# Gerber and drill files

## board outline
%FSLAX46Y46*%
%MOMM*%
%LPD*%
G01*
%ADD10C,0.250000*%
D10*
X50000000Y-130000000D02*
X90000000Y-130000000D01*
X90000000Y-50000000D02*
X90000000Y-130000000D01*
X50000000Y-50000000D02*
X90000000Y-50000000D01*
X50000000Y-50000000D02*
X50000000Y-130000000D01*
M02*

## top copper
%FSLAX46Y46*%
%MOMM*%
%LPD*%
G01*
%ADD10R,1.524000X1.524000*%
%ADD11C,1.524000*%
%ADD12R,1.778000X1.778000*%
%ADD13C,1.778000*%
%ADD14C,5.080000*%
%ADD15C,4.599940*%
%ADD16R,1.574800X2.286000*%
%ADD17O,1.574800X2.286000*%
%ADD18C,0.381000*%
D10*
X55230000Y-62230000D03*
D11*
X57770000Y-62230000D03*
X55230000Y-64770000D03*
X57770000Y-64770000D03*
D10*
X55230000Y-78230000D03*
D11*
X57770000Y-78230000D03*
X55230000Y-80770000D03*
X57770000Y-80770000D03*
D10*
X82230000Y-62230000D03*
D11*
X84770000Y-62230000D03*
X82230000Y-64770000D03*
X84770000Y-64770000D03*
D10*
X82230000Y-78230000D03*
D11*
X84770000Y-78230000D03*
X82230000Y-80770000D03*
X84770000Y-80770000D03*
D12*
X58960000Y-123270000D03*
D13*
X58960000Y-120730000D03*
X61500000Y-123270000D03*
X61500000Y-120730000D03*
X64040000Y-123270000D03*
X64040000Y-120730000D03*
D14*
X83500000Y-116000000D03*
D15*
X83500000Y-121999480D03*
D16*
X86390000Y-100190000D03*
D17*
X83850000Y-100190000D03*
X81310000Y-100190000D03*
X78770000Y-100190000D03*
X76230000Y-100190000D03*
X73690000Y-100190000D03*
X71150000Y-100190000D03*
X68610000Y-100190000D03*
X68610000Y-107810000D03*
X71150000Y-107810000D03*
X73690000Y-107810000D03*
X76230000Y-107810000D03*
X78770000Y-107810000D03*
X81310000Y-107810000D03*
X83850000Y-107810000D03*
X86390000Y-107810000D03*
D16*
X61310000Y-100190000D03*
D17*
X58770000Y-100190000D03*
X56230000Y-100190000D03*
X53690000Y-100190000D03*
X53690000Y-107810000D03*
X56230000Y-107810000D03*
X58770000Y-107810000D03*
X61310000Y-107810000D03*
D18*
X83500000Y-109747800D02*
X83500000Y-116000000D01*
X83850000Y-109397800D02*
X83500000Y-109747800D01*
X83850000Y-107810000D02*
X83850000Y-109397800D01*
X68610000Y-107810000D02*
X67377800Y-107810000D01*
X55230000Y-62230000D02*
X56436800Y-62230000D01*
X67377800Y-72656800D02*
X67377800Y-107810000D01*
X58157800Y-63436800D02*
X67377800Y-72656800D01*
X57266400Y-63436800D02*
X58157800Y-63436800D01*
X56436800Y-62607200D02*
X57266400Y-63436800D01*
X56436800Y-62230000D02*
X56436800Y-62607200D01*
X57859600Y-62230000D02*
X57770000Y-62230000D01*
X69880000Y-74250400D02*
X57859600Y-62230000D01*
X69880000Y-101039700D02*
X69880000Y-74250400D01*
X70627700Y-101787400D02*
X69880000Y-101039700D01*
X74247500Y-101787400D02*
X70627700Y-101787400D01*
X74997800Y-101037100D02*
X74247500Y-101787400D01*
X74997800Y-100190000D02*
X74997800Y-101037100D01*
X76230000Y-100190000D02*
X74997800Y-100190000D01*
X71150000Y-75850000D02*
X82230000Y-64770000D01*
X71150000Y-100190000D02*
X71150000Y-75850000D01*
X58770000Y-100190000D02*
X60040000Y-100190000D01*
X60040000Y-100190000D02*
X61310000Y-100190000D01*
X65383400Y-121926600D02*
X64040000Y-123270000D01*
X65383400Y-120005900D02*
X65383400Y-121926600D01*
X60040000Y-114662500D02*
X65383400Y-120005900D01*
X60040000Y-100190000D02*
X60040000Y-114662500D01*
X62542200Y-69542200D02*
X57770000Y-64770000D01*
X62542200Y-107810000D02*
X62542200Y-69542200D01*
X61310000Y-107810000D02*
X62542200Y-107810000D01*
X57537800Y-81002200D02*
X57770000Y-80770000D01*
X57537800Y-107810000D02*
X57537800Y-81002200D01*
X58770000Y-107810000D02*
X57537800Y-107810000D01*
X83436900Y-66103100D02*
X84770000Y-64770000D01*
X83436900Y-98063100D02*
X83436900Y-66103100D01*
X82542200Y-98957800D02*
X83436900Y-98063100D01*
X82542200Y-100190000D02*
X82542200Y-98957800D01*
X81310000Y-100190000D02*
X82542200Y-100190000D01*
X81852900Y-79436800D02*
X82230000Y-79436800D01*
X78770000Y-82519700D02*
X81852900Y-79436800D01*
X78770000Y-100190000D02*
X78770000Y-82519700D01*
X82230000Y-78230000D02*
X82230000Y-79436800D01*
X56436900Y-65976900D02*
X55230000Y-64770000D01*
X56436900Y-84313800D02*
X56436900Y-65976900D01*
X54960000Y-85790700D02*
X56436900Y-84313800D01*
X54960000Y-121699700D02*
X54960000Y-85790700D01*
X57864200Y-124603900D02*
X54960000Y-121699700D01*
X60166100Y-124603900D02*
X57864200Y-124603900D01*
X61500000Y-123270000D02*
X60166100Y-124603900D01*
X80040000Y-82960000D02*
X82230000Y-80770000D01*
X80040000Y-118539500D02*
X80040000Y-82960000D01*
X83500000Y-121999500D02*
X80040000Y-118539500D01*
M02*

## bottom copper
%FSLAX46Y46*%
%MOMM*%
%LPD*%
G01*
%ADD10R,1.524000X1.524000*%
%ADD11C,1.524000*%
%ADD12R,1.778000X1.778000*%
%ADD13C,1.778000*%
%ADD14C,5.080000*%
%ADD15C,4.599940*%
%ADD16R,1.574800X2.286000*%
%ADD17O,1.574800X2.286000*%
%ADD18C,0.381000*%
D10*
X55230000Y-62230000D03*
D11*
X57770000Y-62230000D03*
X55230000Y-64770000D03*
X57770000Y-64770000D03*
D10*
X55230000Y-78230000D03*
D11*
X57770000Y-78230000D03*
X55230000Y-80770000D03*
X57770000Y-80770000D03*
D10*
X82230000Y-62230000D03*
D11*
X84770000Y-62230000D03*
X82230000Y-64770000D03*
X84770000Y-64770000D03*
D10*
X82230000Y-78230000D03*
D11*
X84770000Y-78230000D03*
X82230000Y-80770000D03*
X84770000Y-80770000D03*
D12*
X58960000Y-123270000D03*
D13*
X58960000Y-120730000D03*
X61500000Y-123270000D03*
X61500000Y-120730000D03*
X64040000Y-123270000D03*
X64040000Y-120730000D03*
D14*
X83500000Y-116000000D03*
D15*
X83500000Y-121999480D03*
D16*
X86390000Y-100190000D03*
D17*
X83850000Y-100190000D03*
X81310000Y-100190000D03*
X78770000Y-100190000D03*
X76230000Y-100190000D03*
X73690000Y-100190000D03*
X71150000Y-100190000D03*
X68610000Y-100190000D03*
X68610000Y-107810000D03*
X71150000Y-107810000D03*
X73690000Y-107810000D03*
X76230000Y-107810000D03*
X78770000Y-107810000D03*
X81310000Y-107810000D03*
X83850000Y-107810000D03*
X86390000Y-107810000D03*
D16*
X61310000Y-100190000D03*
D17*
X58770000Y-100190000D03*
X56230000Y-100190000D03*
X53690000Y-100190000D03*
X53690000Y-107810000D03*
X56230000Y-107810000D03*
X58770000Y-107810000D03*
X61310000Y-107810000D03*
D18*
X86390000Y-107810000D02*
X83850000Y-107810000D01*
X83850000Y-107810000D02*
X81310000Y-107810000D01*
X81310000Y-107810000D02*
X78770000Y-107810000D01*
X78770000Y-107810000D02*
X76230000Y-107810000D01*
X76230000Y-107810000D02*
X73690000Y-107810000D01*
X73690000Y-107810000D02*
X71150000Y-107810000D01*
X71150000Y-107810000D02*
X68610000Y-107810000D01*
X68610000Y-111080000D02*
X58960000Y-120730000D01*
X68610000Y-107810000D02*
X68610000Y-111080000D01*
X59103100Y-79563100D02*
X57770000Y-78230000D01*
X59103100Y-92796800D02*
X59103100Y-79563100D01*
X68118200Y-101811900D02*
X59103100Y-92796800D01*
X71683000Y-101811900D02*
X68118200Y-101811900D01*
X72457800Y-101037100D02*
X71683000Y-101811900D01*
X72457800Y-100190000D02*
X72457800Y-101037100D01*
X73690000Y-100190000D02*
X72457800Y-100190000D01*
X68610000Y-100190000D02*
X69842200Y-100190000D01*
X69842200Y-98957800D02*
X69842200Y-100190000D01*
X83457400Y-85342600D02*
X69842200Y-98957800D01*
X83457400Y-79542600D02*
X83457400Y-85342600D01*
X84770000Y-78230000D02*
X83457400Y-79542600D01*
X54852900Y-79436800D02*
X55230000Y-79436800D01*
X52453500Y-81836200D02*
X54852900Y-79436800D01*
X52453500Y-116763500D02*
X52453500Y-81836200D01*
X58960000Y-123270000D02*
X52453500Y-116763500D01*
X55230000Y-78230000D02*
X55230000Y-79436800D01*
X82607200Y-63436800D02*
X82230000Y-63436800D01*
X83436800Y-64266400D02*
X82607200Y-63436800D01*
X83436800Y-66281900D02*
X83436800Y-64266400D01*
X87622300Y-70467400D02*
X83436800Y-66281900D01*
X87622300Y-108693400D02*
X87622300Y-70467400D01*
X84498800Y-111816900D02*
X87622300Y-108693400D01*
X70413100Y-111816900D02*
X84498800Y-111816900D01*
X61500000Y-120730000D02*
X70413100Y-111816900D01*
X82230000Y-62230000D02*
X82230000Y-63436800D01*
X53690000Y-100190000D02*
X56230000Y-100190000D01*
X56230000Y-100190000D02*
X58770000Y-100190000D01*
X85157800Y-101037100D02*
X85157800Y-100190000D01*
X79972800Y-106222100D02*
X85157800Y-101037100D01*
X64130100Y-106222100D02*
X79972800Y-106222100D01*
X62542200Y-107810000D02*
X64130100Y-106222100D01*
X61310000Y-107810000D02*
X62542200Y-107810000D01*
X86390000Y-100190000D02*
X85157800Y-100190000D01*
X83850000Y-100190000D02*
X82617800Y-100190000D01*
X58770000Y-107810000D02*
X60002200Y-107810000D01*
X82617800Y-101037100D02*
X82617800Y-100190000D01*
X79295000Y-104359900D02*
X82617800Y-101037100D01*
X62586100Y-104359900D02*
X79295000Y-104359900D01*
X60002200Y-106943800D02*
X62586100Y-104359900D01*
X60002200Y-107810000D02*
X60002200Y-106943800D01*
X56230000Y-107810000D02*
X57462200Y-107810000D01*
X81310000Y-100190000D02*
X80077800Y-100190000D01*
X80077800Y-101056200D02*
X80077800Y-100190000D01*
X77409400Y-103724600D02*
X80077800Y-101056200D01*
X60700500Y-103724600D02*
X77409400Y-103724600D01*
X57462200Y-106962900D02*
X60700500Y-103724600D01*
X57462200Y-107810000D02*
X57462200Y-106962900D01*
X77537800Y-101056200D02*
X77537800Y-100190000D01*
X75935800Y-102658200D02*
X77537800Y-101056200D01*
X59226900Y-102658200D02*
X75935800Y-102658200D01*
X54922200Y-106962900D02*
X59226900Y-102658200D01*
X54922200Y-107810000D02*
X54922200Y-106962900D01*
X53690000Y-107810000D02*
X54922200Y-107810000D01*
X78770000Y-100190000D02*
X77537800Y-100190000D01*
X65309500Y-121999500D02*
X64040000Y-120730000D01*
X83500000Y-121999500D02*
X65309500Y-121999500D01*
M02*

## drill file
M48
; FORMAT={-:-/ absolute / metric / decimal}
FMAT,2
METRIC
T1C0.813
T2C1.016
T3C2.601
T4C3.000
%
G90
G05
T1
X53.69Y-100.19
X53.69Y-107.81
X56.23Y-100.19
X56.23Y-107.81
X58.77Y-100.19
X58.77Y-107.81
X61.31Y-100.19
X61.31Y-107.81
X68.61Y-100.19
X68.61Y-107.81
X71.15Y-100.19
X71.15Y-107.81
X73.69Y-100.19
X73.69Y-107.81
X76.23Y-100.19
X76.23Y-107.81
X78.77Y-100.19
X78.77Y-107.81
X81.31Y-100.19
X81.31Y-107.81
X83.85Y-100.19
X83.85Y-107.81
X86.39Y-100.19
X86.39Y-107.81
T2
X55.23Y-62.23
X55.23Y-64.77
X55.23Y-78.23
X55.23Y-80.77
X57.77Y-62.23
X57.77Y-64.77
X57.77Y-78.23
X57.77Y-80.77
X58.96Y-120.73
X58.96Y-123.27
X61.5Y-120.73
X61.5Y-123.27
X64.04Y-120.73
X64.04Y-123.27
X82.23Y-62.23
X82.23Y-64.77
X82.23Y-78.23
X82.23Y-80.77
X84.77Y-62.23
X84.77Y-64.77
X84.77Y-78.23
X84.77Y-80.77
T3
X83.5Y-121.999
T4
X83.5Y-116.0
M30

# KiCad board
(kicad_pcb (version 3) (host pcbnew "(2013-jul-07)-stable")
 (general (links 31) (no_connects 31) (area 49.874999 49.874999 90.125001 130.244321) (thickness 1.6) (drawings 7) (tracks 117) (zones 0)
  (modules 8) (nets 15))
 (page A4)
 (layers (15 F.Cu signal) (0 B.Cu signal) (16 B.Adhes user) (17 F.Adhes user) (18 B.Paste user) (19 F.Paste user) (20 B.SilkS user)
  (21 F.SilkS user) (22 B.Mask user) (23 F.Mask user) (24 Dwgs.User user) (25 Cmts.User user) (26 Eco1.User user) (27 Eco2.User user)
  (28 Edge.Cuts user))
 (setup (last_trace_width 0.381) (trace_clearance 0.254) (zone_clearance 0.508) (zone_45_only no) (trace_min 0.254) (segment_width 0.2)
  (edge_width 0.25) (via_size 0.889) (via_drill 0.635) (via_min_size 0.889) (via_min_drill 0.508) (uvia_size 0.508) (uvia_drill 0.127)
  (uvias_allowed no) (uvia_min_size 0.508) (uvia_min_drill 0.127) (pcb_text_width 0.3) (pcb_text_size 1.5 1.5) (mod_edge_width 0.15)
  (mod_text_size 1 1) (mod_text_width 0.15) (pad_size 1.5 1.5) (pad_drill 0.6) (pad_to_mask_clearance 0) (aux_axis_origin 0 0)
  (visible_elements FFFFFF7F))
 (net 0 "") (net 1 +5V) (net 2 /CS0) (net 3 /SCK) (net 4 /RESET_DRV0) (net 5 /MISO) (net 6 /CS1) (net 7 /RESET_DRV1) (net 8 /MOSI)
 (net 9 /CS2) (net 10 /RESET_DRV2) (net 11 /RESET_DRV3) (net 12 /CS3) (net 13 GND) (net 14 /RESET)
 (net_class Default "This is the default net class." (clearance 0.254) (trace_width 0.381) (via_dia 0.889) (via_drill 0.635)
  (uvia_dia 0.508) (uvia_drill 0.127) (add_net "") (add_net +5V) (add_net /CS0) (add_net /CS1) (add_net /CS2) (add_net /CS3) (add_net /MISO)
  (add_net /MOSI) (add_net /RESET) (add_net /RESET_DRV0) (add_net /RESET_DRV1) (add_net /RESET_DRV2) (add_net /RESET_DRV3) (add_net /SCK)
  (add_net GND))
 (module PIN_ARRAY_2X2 (layer F.Cu) (at 56.5 63.5 270)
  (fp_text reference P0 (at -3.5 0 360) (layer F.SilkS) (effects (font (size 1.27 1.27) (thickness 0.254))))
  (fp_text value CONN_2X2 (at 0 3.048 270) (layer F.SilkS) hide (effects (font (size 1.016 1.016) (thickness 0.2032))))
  (pad 1 thru_hole rect (at -1.27 1.27 270) (size 1.524 1.524) (drill 1.016) (layers *.Cu *.Mask F.SilkS) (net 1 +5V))
  (pad 2 thru_hole circle (at -1.27 -1.27 270) (size 1.524 1.524) (drill 1.016) (layers *.Cu *.Mask F.SilkS) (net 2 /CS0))
  (pad 3 thru_hole circle (at 1.27 1.27 270) (size 1.524 1.524) (drill 1.016) (layers *.Cu *.Mask F.SilkS) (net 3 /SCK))
  (pad 4 thru_hole circle (at 1.27 -1.27 270) (size 1.524 1.524) (drill 1.016) (layers *.Cu *.Mask F.SilkS) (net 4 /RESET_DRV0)))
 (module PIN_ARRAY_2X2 (layer F.Cu) (at 56.5 79.5 270)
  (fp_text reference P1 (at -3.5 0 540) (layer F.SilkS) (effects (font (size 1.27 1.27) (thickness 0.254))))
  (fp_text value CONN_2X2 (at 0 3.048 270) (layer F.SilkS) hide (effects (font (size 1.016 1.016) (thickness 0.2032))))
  (pad 1 thru_hole rect (at -1.27 1.27 270) (size 1.524 1.524) (drill 1.016) (layers *.Cu *.Mask F.SilkS) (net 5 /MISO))
  (pad 2 thru_hole circle (at -1.27 -1.27 270) (size 1.524 1.524) (drill 1.016) (layers *.Cu *.Mask F.SilkS) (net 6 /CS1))
  (pad 3 thru_hole circle (at 1.27 1.27 270) (size 1.524 1.524) (drill 1.016) (layers *.Cu *.Mask F.SilkS))
  (pad 4 thru_hole circle (at 1.27 -1.27 270) (size 1.524 1.524) (drill 1.016) (layers *.Cu *.Mask F.SilkS) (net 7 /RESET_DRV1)))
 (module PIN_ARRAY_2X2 (layer F.Cu) (at 83.5 63.5 270)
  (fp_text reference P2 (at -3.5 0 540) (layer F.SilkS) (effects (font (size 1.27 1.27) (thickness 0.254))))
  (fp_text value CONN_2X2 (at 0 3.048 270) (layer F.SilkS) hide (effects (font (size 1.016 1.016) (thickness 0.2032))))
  (pad 1 thru_hole rect (at -1.27 1.27 270) (size 1.524 1.524) (drill 1.016) (layers *.Cu *.Mask F.SilkS) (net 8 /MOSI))
  (pad 2 thru_hole circle (at -1.27 -1.27 270) (size 1.524 1.524) (drill 1.016) (layers *.Cu *.Mask F.SilkS))
  (pad 3 thru_hole circle (at 1.27 1.27 270) (size 1.524 1.524) (drill 1.016) (layers *.Cu *.Mask F.SilkS) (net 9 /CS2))
  (pad 4 thru_hole circle (at 1.27 -1.27 270) (size 1.524 1.524) (drill 1.016) (layers *.Cu *.Mask F.SilkS) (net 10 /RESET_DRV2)))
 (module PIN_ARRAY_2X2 (layer F.Cu) (at 83.5 79.5 270)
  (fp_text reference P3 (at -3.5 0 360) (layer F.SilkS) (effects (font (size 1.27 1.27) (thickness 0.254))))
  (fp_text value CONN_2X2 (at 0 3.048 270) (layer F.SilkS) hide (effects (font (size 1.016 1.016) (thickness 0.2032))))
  (pad 1 thru_hole rect (at -1.27 1.27 270) (size 1.524 1.524) (drill 1.016) (layers *.Cu *.Mask F.SilkS) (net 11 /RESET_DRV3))
  (pad 2 thru_hole circle (at -1.27 -1.27 270) (size 1.524 1.524) (drill 1.016) (layers *.Cu *.Mask F.SilkS) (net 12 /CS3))
  (pad 3 thru_hole circle (at 1.27 1.27 270) (size 1.524 1.524) (drill 1.016) (layers *.Cu *.Mask F.SilkS) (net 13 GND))
  (pad 4 thru_hole circle (at 1.27 -1.27 270) (size 1.524 1.524) (drill 1.016) (layers *.Cu *.Mask F.SilkS)))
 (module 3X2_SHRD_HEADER (layer F.Cu) (at 61.5 122)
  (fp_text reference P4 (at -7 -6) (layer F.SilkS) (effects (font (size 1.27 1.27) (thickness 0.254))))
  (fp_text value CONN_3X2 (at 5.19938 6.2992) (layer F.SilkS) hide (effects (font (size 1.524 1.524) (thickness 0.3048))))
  (pad 1 thru_hole rect (at -2.54 1.27) (size 1.778 1.778) (drill 1.016) (layers *.Cu *.Mask F.SilkS) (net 5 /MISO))
  (pad 2 thru_hole circle (at -2.54 -1.27) (size 1.778 1.778) (drill 1.016) (layers *.Cu *.Mask F.SilkS) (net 1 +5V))
  (pad 3 thru_hole circle (at 0 1.27) (size 1.778 1.778) (drill 1.016) (layers *.Cu *.Mask F.SilkS) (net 3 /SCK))
  (pad 4 thru_hole circle (at 0 -1.27) (size 1.778 1.778) (drill 1.016) (layers *.Cu *.Mask F.SilkS) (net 8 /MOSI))
  (pad 5 thru_hole circle (at 2.54 1.27) (size 1.778 1.778) (drill 1.016) (layers *.Cu *.Mask F.SilkS) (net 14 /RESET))
  (pad 6 thru_hole circle (at 2.54 -1.27) (size 1.778 1.778) (drill 1.016) (layers *.Cu *.Mask F.SilkS) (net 13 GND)))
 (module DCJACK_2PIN (layer F.Cu) (at 83.5 116 270)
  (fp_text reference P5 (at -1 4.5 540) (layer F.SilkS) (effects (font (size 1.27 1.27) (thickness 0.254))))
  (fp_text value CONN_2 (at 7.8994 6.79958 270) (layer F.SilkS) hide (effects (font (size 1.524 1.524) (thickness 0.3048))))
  (pad 1 thru_hole circle (at 0 0 270) (size 5.08 5.08) (drill 2.99974) (layers *.Cu *.Mask F.SilkS) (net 1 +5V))
  (pad 2 thru_hole circle (at 5.99948 0 270) (size 4.59994 4.59994) (drill 2.60096) (layers *.Cu *.Mask F.SilkS) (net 13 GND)))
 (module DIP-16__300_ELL (layer F.Cu) (at 77.5 104 180)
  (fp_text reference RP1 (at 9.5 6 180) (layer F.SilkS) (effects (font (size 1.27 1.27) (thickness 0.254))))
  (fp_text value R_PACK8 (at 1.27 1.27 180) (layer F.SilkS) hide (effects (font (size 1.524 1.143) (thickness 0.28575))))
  (pad 1 thru_hole rect (at -8.89 3.81 180) (size 1.5748 2.286) (drill 0.8128) (layers *.Cu *.Mask F.SilkS) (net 4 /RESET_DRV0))
  (pad 2 thru_hole oval (at -6.35 3.81 180) (size 1.5748 2.286) (drill 0.8128) (layers *.Cu *.Mask F.SilkS) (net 7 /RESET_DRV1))
  (pad 3 thru_hole oval (at -3.81 3.81 180) (size 1.5748 2.286) (drill 0.8128) (layers *.Cu *.Mask F.SilkS) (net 10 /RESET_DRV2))
  (pad 4 thru_hole oval (at -1.27 3.81 180) (size 1.5748 2.286) (drill 0.8128) (layers *.Cu *.Mask F.SilkS) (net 11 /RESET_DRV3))
  (pad 5 thru_hole oval (at 1.27 3.81 180) (size 1.5748 2.286) (drill 0.8128) (layers *.Cu *.Mask F.SilkS) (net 2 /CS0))
  (pad 6 thru_hole oval (at 3.81 3.81 180) (size 1.5748 2.286) (drill 0.8128) (layers *.Cu *.Mask F.SilkS) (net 6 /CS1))
  (pad 7 thru_hole oval (at 6.35 3.81 180) (size 1.5748 2.286) (drill 0.8128) (layers *.Cu *.Mask F.SilkS) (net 9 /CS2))
  (pad 8 thru_hole oval (at 8.89 3.81 180) (size 1.5748 2.286) (drill 0.8128) (layers *.Cu *.Mask F.SilkS) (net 12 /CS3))
  (pad 9 thru_hole oval (at 8.89 -3.81 180) (size 1.5748 2.286) (drill 0.8128) (layers *.Cu *.Mask F.SilkS) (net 1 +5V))
  (pad 10 thru_hole oval (at 6.35 -3.81 180) (size 1.5748 2.286) (drill 0.8128) (layers *.Cu *.Mask F.SilkS) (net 1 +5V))
  (pad 11 thru_hole oval (at 3.81 -3.81 180) (size 1.5748 2.286) (drill 0.8128) (layers *.Cu *.Mask F.SilkS) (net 1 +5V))
  (pad 12 thru_hole oval (at 1.27 -3.81 180) (size 1.5748 2.286) (drill 0.8128) (layers *.Cu *.Mask F.SilkS) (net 1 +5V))
  (pad 13 thru_hole oval (at -1.27 -3.81 180) (size 1.5748 2.286) (drill 0.8128) (layers *.Cu *.Mask F.SilkS) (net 1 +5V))
  (pad 14 thru_hole oval (at -3.81 -3.81 180) (size 1.5748 2.286) (drill 0.8128) (layers *.Cu *.Mask F.SilkS) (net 1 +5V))
  (pad 15 thru_hole oval (at -6.35 -3.81 180) (size 1.5748 2.286) (drill 0.8128) (layers *.Cu *.Mask F.SilkS) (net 1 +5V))
  (pad 16 thru_hole oval (at -8.89 -3.81 180) (size 1.5748 2.286) (drill 0.8128) (layers *.Cu *.Mask F.SilkS) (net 1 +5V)))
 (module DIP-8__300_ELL (layer F.Cu) (at 57.5 104 180)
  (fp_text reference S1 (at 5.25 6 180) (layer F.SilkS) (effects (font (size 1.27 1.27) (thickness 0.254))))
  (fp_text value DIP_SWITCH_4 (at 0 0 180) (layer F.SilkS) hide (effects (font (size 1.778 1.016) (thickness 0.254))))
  (pad 1 thru_hole rect (at -3.81 3.81 180) (size 1.5748 2.286) (drill 0.8128) (layers *.Cu *.Mask F.SilkS) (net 14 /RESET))
  (pad 2 thru_hole oval (at -1.27 3.81 180) (size 1.5748 2.286) (drill 0.8128) (layers *.Cu *.Mask F.SilkS) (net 14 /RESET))
  (pad 3 thru_hole oval (at 1.27 3.81 180) (size 1.5748 2.286) (drill 0.8128) (layers *.Cu *.Mask F.SilkS) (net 14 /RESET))
  (pad 4 thru_hole oval (at 3.81 3.81 180) (size 1.5748 2.286) (drill 0.8128) (layers *.Cu *.Mask F.SilkS) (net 14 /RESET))
  (pad 5 thru_hole oval (at 3.81 -3.81 180) (size 1.5748 2.286) (drill 0.8128) (layers *.Cu *.Mask F.SilkS) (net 11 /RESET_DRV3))
  (pad 6 thru_hole oval (at 1.27 -3.81 180) (size 1.5748 2.286) (drill 0.8128) (layers *.Cu *.Mask F.SilkS) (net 10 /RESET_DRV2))
  (pad 7 thru_hole oval (at -1.27 -3.81 180) (size 1.5748 2.286) (drill 0.8128) (layers *.Cu *.Mask F.SilkS) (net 7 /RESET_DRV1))
  (pad 8 thru_hole oval (at -3.81 -3.81 180) (size 1.5748 2.286) (drill 0.8128) (layers *.Cu *.Mask F.SilkS) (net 4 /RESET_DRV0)))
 (gr_line (start 50 130) (end 90 130) (angle 90) (layer Edge.Cuts) (width 0.25))
 (gr_line (start 90 50) (end 90 130) (angle 90) (layer Edge.Cuts) (width 0.25))
 (gr_line (start 50 50) (end 90 50) (angle 90) (layer Edge.Cuts) (width 0.25))
 (gr_line (start 50 50) (end 50 130) (angle 90) (layer Edge.Cuts) (width 0.25))
 (segment (start 86.39 107.81) (end 83.85 107.81) (width 0.381) (layer B.Cu) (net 1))
 (segment (start 83.85 107.81) (end 81.31 107.81) (width 0.381) (layer B.Cu) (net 1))
 (segment (start 81.31 107.81) (end 78.77 107.81) (width 0.381) (layer B.Cu) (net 1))
 (segment (start 78.77 107.81) (end 76.23 107.81) (width 0.381) (layer B.Cu) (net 1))
 (segment (start 76.23 107.81) (end 73.69 107.81) (width 0.381) (layer B.Cu) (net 1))
 (segment (start 73.69 107.81) (end 71.15 107.81) (width 0.381) (layer B.Cu) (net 1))
 (segment (start 83.5 109.7478) (end 83.5 116) (width 0.381) (layer F.Cu) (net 1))
 (segment (start 83.85 109.3978) (end 83.5 109.7478) (width 0.381) (layer F.Cu) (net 1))
 (segment (start 83.85 107.81) (end 83.85 109.3978) (width 0.381) (layer F.Cu) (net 1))
 (segment (start 71.15 107.81) (end 68.61 107.81) (width 0.381) (layer B.Cu) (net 1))
 (segment (start 68.61 111.08) (end 58.96 120.73) (width 0.381) (layer B.Cu) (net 1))
 (segment (start 68.61 107.81) (end 68.61 111.08) (width 0.381) (layer B.Cu) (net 1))
 (segment (start 68.61 107.81) (end 67.3778 107.81) (width 0.381) (layer F.Cu) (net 1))
 (segment (start 55.23 62.23) (end 56.4368 62.23) (width 0.381) (layer F.Cu) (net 1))
 (segment (start 67.3778 72.6568) (end 67.3778 107.81) (width 0.381) (layer F.Cu) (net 1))
 (segment (start 58.1578 63.4368) (end 67.3778 72.6568) (width 0.381) (layer F.Cu) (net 1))
 (segment (start 57.2664 63.4368) (end 58.1578 63.4368) (width 0.381) (layer F.Cu) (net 1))
 (segment (start 56.4368 62.6072) (end 57.2664 63.4368) (width 0.381) (layer F.Cu) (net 1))
 (segment (start 56.4368 62.23) (end 56.4368 62.6072) (width 0.381) (layer F.Cu) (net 1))
 (segment (start 57.8596 62.23) (end 57.77 62.23) (width 0.381) (layer F.Cu) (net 2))
 (segment (start 69.88 74.2504) (end 57.8596 62.23) (width 0.381) (layer F.Cu) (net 2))
 (segment (start 69.88 101.0397) (end 69.88 74.2504) (width 0.381) (layer F.Cu) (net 2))
 (segment (start 70.6277 101.7874) (end 69.88 101.0397) (width 0.381) (layer F.Cu) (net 2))
 (segment (start 74.2475 101.7874) (end 70.6277 101.7874) (width 0.381) (layer F.Cu) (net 2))
 (segment (start 74.9978 101.0371) (end 74.2475 101.7874) (width 0.381) (layer F.Cu) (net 2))
 (segment (start 74.9978 100.19) (end 74.9978 101.0371) (width 0.381) (layer F.Cu) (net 2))
 (segment (start 76.23 100.19) (end 74.9978 100.19) (width 0.381) (layer F.Cu) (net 2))
 (segment (start 59.1031 79.5631) (end 57.77 78.23) (width 0.381) (layer B.Cu) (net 6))
 (segment (start 59.1031 92.7968) (end 59.1031 79.5631) (width 0.381) (layer B.Cu) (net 6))
 (segment (start 68.1182 101.8119) (end 59.1031 92.7968) (width 0.381) (layer B.Cu) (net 6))
 (segment (start 71.683 101.8119) (end 68.1182 101.8119) (width 0.381) (layer B.Cu) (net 6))
 (segment (start 72.4578 101.0371) (end 71.683 101.8119) (width 0.381) (layer B.Cu) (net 6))
 (segment (start 72.4578 100.19) (end 72.4578 101.0371) (width 0.381) (layer B.Cu) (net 6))
 (segment (start 73.69 100.19) (end 72.4578 100.19) (width 0.381) (layer B.Cu) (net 6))
 (segment (start 71.15 75.85) (end 82.23 64.77) (width 0.381) (layer F.Cu) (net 9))
 (segment (start 71.15 100.19) (end 71.15 75.85) (width 0.381) (layer F.Cu) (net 9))
 (segment (start 68.61 100.19) (end 69.8422 100.19) (width 0.381) (layer B.Cu) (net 12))
 (segment (start 69.8422 98.9578) (end 69.8422 100.19) (width 0.381) (layer B.Cu) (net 12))
 (segment (start 83.4574 85.3426) (end 69.8422 98.9578) (width 0.381) (layer B.Cu) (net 12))
 (segment (start 83.4574 79.5426) (end 83.4574 85.3426) (width 0.381) (layer B.Cu) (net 12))
 (segment (start 84.77 78.23) (end 83.4574 79.5426) (width 0.381) (layer B.Cu) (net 12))
 (segment (start 54.8529 79.4368) (end 55.23 79.4368) (width 0.381) (layer B.Cu) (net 5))
 (segment (start 52.4535 81.8362) (end 54.8529 79.4368) (width 0.381) (layer B.Cu) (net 5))
 (segment (start 52.4535 116.7635) (end 52.4535 81.8362) (width 0.381) (layer B.Cu) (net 5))
 (segment (start 58.96 123.27) (end 52.4535 116.7635) (width 0.381) (layer B.Cu) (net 5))
 (segment (start 55.23 78.23) (end 55.23 79.4368) (width 0.381) (layer B.Cu) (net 5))
 (segment (start 82.6072 63.4368) (end 82.23 63.4368) (width 0.381) (layer B.Cu) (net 8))
 (segment (start 83.4368 64.2664) (end 82.6072 63.4368) (width 0.381) (layer B.Cu) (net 8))
 (segment (start 83.4368 66.2819) (end 83.4368 64.2664) (width 0.381) (layer B.Cu) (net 8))
 (segment (start 87.6223 70.4674) (end 83.4368 66.2819) (width 0.381) (layer B.Cu) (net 8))
 (segment (start 87.6223 108.6934) (end 87.6223 70.4674) (width 0.381) (layer B.Cu) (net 8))
 (segment (start 84.4988 111.8169) (end 87.6223 108.6934) (width 0.381) (layer B.Cu) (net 8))
 (segment (start 70.4131 111.8169) (end 84.4988 111.8169) (width 0.381) (layer B.Cu) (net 8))
 (segment (start 61.5 120.73) (end 70.4131 111.8169) (width 0.381) (layer B.Cu) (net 8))
 (segment (start 82.23 62.23) (end 82.23 63.4368) (width 0.381) (layer B.Cu) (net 8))
 (segment (start 53.69 100.19) (end 56.23 100.19) (width 0.381) (layer B.Cu) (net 14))
 (segment (start 56.23 100.19) (end 58.77 100.19) (width 0.381) (layer B.Cu) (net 14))
 (segment (start 58.77 100.19) (end 60.04 100.19) (width 0.381) (layer F.Cu) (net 14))
 (segment (start 60.04 100.19) (end 61.31 100.19) (width 0.381) (layer F.Cu) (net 14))
 (segment (start 65.3834 121.9266) (end 64.04 123.27) (width 0.381) (layer F.Cu) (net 14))
 (segment (start 65.3834 120.0059) (end 65.3834 121.9266) (width 0.381) (layer F.Cu) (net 14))
 (segment (start 60.04 114.6625) (end 65.3834 120.0059) (width 0.381) (layer F.Cu) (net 14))
 (segment (start 60.04 100.19) (end 60.04 114.6625) (width 0.381) (layer F.Cu) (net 14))
 (segment (start 62.5422 69.5422) (end 57.77 64.77) (width 0.381) (layer F.Cu) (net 4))
 (segment (start 62.5422 107.81) (end 62.5422 69.5422) (width 0.381) (layer F.Cu) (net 4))
 (segment (start 61.31 107.81) (end 62.5422 107.81) (width 0.381) (layer F.Cu) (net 4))
 (segment (start 85.1578 101.0371) (end 85.1578 100.19) (width 0.381) (layer B.Cu) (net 4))
 (segment (start 79.9728 106.2221) (end 85.1578 101.0371) (width 0.381) (layer B.Cu) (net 4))
 (segment (start 64.1301 106.2221) (end 79.9728 106.2221) (width 0.381) (layer B.Cu) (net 4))
 (segment (start 62.5422 107.81) (end 64.1301 106.2221) (width 0.381) (layer B.Cu) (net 4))
 (segment (start 61.31 107.81) (end 62.5422 107.81) (width 0.381) (layer B.Cu) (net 4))
 (segment (start 86.39 100.19) (end 85.1578 100.19) (width 0.381) (layer B.Cu) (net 4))
 (segment (start 57.5378 81.0022) (end 57.77 80.77) (width 0.381) (layer F.Cu) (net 7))
 (segment (start 57.5378 107.81) (end 57.5378 81.0022) (width 0.381) (layer F.Cu) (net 7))
 (segment (start 58.77 107.81) (end 57.5378 107.81) (width 0.381) (layer F.Cu) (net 7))
 (segment (start 83.85 100.19) (end 82.6178 100.19) (width 0.381) (layer B.Cu) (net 7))
 (segment (start 58.77 107.81) (end 60.0022 107.81) (width 0.381) (layer B.Cu) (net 7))
 (segment (start 82.6178 101.0371) (end 82.6178 100.19) (width 0.381) (layer B.Cu) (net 7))
 (segment (start 79.295 104.3599) (end 82.6178 101.0371) (width 0.381) (layer B.Cu) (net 7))
 (segment (start 62.5861 104.3599) (end 79.295 104.3599) (width 0.381) (layer B.Cu) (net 7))
 (segment (start 60.0022 106.9438) (end 62.5861 104.3599) (width 0.381) (layer B.Cu) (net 7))
 (segment (start 60.0022 107.81) (end 60.0022 106.9438) (width 0.381) (layer B.Cu) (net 7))
 (segment (start 56.23 107.81) (end 57.4622 107.81) (width 0.381) (layer B.Cu) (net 10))
 (segment (start 81.31 100.19) (end 80.0778 100.19) (width 0.381) (layer B.Cu) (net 10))
 (segment (start 83.4369 66.1031) (end 84.77 64.77) (width 0.381) (layer F.Cu) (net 10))
 (segment (start 83.4369 98.0631) (end 83.4369 66.1031) (width 0.381) (layer F.Cu) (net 10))
 (segment (start 82.5422 98.9578) (end 83.4369 98.0631) (width 0.381) (layer F.Cu) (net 10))
 (segment (start 82.5422 100.19) (end 82.5422 98.9578) (width 0.381) (layer F.Cu) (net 10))
 (segment (start 81.31 100.19) (end 82.5422 100.19) (width 0.381) (layer F.Cu) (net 10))
 (segment (start 80.0778 101.0562) (end 80.0778 100.19) (width 0.381) (layer B.Cu) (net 10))
 (segment (start 77.4094 103.7246) (end 80.0778 101.0562) (width 0.381) (layer B.Cu) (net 10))
 (segment (start 60.7005 103.7246) (end 77.4094 103.7246) (width 0.381) (layer B.Cu) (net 10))
 (segment (start 57.4622 106.9629) (end 60.7005 103.7246) (width 0.381) (layer B.Cu) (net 10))
 (segment (start 57.4622 107.81) (end 57.4622 106.9629) (width 0.381) (layer B.Cu) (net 10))
 (segment (start 81.8529 79.4368) (end 82.23 79.4368) (width 0.381) (layer F.Cu) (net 11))
 (segment (start 78.77 82.5197) (end 81.8529 79.4368) (width 0.381) (layer F.Cu) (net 11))
 (segment (start 78.77 100.19) (end 78.77 82.5197) (width 0.381) (layer F.Cu) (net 11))
 (segment (start 82.23 78.23) (end 82.23 79.4368) (width 0.381) (layer F.Cu) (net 11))
 (segment (start 77.5378 101.0562) (end 77.5378 100.19) (width 0.381) (layer B.Cu) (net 11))
 (segment (start 75.9358 102.6582) (end 77.5378 101.0562) (width 0.381) (layer B.Cu) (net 11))
 (segment (start 59.2269 102.6582) (end 75.9358 102.6582) (width 0.381) (layer B.Cu) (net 11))
 (segment (start 54.9222 106.9629) (end 59.2269 102.6582) (width 0.381) (layer B.Cu) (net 11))
 (segment (start 54.9222 107.81) (end 54.9222 106.9629) (width 0.381) (layer B.Cu) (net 11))
 (segment (start 53.69 107.81) (end 54.9222 107.81) (width 0.381) (layer B.Cu) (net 11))
 (segment (start 78.77 100.19) (end 77.5378 100.19) (width 0.381) (layer B.Cu) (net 11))
 (segment (start 56.4369 65.9769) (end 55.23 64.77) (width 0.381) (layer F.Cu) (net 3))
 (segment (start 56.4369 84.3138) (end 56.4369 65.9769) (width 0.381) (layer F.Cu) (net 3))
 (segment (start 54.96 85.7907) (end 56.4369 84.3138) (width 0.381) (layer F.Cu) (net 3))
 (segment (start 54.96 121.6997) (end 54.96 85.7907) (width 0.381) (layer F.Cu) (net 3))
 (segment (start 57.8642 124.6039) (end 54.96 121.6997) (width 0.381) (layer F.Cu) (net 3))
 (segment (start 60.1661 124.6039) (end 57.8642 124.6039) (width 0.381) (layer F.Cu) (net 3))
 (segment (start 61.5 123.27) (end 60.1661 124.6039) (width 0.381) (layer F.Cu) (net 3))
 (segment (start 65.3095 121.9995) (end 64.04 120.73) (width 0.381) (layer B.Cu) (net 13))
 (segment (start 83.5 121.9995) (end 65.3095 121.9995) (width 0.381) (layer B.Cu) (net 13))
 (segment (start 80.04 82.96) (end 82.23 80.77) (width 0.381) (layer F.Cu) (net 13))
 (segment (start 80.04 118.5395) (end 80.04 82.96) (width 0.381) (layer F.Cu) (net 13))
 (segment (start 83.5 121.9995) (end 80.04 118.5395) (width 0.381) (layer F.Cu) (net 13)))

